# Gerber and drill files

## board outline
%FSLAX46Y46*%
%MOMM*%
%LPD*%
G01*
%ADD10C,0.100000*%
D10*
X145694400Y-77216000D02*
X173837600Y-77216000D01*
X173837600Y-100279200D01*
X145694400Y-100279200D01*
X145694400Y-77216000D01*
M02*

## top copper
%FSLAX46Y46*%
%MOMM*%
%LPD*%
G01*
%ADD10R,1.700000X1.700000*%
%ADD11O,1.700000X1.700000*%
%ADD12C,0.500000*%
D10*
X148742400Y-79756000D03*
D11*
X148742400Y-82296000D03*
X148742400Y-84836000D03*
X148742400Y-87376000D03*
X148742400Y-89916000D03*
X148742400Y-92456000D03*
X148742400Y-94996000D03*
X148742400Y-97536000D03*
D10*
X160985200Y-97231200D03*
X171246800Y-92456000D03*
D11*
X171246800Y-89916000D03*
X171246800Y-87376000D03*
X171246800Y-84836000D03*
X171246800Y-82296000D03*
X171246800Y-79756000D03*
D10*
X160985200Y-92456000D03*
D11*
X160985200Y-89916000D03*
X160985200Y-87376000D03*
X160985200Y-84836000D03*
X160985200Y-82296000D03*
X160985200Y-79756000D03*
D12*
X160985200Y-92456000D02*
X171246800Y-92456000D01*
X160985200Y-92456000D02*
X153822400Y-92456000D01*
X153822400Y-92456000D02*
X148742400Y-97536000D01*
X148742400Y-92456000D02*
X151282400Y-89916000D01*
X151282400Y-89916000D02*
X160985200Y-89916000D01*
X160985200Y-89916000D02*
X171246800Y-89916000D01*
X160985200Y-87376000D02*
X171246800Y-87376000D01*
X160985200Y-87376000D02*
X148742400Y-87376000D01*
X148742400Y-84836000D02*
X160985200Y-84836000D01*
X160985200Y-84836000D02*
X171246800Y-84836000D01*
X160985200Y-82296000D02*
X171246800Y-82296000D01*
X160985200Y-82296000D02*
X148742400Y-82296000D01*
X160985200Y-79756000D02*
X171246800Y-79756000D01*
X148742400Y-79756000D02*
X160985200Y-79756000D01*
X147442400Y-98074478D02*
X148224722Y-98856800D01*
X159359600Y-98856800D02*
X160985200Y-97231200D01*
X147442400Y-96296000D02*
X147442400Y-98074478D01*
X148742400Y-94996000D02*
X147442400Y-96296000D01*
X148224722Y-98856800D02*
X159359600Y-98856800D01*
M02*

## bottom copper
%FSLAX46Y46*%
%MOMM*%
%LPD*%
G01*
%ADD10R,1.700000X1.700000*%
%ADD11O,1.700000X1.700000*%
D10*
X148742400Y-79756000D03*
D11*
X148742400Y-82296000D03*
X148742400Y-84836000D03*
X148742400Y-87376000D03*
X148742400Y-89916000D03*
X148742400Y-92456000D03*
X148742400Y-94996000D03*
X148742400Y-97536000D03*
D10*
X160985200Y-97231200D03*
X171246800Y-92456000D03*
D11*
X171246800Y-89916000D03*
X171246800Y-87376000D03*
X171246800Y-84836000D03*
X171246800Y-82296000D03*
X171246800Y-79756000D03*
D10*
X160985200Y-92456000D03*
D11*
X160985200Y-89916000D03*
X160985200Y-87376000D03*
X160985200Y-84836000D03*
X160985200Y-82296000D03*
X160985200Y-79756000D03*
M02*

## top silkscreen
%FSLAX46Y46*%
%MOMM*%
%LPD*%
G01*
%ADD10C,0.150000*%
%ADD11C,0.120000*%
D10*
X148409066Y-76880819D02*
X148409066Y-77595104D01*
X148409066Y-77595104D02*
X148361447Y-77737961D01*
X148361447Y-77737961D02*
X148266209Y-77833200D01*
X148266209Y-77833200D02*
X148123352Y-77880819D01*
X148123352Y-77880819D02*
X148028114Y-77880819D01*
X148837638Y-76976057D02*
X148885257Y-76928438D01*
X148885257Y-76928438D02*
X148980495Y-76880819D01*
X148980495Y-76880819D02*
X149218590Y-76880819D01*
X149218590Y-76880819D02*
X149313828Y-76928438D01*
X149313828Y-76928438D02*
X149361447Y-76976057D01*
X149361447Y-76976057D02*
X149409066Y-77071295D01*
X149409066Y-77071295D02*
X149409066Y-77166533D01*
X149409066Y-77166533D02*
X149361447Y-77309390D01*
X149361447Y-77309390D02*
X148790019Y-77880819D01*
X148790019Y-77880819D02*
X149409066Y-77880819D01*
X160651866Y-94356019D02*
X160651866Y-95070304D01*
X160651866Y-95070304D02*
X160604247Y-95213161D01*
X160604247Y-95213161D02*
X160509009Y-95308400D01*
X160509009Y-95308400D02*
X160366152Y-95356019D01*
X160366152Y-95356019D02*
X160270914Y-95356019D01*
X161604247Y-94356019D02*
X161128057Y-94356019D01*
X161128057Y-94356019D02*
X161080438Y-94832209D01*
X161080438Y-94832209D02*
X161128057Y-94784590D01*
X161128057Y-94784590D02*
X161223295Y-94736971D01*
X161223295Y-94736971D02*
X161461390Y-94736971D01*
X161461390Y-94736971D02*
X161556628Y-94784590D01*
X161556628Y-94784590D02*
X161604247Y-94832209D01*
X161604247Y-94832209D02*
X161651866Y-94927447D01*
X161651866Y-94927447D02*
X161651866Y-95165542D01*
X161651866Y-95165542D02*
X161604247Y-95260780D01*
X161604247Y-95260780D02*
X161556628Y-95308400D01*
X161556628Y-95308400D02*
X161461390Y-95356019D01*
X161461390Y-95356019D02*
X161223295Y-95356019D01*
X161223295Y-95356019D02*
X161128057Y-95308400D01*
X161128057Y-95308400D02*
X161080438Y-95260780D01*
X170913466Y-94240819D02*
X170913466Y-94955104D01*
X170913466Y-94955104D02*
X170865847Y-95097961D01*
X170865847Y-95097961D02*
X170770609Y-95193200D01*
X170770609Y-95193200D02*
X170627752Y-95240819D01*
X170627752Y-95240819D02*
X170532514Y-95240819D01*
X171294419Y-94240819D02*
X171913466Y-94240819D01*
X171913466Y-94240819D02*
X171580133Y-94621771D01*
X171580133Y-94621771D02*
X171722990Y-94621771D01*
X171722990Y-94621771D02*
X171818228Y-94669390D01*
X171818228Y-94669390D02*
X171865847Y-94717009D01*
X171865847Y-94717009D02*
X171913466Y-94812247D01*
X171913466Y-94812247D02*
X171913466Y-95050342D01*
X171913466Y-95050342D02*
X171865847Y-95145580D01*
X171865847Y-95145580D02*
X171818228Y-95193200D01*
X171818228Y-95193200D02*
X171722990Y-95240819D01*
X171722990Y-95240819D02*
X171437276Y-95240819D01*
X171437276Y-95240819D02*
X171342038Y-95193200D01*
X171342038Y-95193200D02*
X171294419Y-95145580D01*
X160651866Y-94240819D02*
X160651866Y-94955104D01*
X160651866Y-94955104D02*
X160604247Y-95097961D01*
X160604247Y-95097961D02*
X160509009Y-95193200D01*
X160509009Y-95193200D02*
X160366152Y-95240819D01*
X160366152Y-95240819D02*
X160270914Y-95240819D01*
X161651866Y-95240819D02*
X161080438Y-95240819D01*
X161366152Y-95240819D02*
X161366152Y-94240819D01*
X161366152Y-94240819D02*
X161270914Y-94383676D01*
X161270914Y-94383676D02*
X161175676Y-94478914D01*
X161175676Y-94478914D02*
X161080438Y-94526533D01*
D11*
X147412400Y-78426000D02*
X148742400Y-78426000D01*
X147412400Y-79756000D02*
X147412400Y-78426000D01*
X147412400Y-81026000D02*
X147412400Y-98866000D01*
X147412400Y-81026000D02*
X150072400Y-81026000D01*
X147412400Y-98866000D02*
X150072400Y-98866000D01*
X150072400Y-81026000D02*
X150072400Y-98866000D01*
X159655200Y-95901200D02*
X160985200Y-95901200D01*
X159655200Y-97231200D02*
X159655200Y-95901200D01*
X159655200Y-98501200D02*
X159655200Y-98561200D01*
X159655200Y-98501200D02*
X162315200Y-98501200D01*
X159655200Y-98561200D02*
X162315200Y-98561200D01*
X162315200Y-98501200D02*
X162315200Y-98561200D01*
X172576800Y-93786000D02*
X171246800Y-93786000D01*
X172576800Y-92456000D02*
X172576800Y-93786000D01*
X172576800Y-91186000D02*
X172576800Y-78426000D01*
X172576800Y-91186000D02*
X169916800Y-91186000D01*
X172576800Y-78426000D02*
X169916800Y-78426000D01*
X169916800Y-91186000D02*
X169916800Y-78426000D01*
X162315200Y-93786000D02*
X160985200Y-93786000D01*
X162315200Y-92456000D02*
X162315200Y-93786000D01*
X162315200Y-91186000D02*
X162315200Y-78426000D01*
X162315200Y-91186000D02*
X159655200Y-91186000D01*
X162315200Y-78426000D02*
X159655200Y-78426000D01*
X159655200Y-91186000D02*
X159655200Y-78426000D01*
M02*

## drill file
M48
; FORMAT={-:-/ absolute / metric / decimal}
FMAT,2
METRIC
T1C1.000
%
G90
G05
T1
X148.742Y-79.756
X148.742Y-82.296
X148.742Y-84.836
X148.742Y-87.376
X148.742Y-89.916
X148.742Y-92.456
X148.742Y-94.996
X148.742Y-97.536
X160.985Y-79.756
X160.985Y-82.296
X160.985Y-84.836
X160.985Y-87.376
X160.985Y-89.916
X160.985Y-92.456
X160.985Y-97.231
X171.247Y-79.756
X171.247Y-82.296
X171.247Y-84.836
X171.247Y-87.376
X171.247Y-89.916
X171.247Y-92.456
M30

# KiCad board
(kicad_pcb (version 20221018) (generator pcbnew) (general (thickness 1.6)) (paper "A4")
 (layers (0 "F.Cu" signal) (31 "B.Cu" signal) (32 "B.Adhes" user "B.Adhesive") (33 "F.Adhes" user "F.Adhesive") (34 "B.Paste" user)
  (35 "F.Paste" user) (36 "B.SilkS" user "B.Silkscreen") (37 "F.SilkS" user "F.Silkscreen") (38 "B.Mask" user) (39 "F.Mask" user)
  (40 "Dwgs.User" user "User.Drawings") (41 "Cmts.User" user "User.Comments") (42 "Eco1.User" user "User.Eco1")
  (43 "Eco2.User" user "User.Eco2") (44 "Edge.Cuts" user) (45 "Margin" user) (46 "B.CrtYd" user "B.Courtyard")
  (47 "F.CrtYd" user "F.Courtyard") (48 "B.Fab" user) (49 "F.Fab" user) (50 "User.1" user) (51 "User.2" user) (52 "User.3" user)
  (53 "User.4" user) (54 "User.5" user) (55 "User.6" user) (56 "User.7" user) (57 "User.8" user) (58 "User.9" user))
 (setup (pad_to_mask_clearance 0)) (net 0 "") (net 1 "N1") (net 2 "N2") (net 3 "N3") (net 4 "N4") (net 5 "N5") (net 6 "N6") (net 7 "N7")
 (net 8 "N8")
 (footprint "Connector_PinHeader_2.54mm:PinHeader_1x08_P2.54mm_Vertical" (layer "F.Cu") (at 148.7424 79.756)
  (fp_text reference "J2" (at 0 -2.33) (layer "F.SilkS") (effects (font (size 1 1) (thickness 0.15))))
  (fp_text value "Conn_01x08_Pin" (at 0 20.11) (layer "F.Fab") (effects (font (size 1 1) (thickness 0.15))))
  (fp_line (start -1.33 -1.33) (end 0 -1.33) (stroke (width 0.12) (type solid)) (layer "F.SilkS"))
  (fp_line (start -1.33 0) (end -1.33 -1.33) (stroke (width 0.12) (type solid)) (layer "F.SilkS"))
  (fp_line (start -1.33 1.27) (end -1.33 19.11) (stroke (width 0.12) (type solid)) (layer "F.SilkS"))
  (fp_line (start -1.33 1.27) (end 1.33 1.27) (stroke (width 0.12) (type solid)) (layer "F.SilkS"))
  (fp_line (start -1.33 19.11) (end 1.33 19.11) (stroke (width 0.12) (type solid)) (layer "F.SilkS"))
  (fp_line (start 1.33 1.27) (end 1.33 19.11) (stroke (width 0.12) (type solid)) (layer "F.SilkS"))
  (pad "1" thru_hole rect (at 0 0) (size 1.7 1.7) (drill 1) (layers "*.Cu" "*.Mask") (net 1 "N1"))
  (pad "2" thru_hole oval (at 0 2.54) (size 1.7 1.7) (drill 1) (layers "*.Cu" "*.Mask") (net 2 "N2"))
  (pad "3" thru_hole oval (at 0 5.08) (size 1.7 1.7) (drill 1) (layers "*.Cu" "*.Mask") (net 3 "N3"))
  (pad "4" thru_hole oval (at 0 7.62) (size 1.7 1.7) (drill 1) (layers "*.Cu" "*.Mask") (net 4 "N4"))
  (pad "5" thru_hole oval (at 0 10.16) (size 1.7 1.7) (drill 1) (layers "*.Cu" "*.Mask") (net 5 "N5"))
  (pad "6" thru_hole oval (at 0 12.7) (size 1.7 1.7) (drill 1) (layers "*.Cu" "*.Mask") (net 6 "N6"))
  (pad "7" thru_hole oval (at 0 15.24) (size 1.7 1.7) (drill 1) (layers "*.Cu" "*.Mask") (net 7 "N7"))
  (pad "8" thru_hole oval (at 0 17.78) (size 1.7 1.7) (drill 1) (layers "*.Cu" "*.Mask") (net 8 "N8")))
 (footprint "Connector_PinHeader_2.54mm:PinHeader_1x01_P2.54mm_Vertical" (layer "F.Cu") (at 160.9852 97.2312)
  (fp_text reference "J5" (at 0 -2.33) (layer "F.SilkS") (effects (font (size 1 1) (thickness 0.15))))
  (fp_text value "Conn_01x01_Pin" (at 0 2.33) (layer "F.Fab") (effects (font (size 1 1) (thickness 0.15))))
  (fp_line (start -1.33 -1.33) (end 0 -1.33) (stroke (width 0.12) (type solid)) (layer "F.SilkS"))
  (fp_line (start -1.33 0) (end -1.33 -1.33) (stroke (width 0.12) (type solid)) (layer "F.SilkS"))
  (fp_line (start -1.33 1.27) (end -1.33 1.33) (stroke (width 0.12) (type solid)) (layer "F.SilkS"))
  (fp_line (start -1.33 1.27) (end 1.33 1.27) (stroke (width 0.12) (type solid)) (layer "F.SilkS"))
  (fp_line (start -1.33 1.33) (end 1.33 1.33) (stroke (width 0.12) (type solid)) (layer "F.SilkS"))
  (fp_line (start 1.33 1.27) (end 1.33 1.33) (stroke (width 0.12) (type solid)) (layer "F.SilkS"))
  (pad "1" thru_hole rect (at 0 0) (size 1.7 1.7) (drill 1) (layers "*.Cu" "*.Mask") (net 7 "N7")))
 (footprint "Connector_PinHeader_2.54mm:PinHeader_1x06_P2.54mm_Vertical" (layer "F.Cu") (at 171.2468 92.456 180)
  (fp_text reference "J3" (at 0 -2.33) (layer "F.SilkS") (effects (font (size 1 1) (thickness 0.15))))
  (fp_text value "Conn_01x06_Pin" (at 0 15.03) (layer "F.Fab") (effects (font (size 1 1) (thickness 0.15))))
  (fp_line (start -1.33 -1.33) (end 0 -1.33) (stroke (width 0.12) (type solid)) (layer "F.SilkS"))
  (fp_line (start -1.33 0) (end -1.33 -1.33) (stroke (width 0.12) (type solid)) (layer "F.SilkS"))
  (fp_line (start -1.33 1.27) (end -1.33 14.03) (stroke (width 0.12) (type solid)) (layer "F.SilkS"))
  (fp_line (start -1.33 1.27) (end 1.33 1.27) (stroke (width 0.12) (type solid)) (layer "F.SilkS"))
  (fp_line (start -1.33 14.03) (end 1.33 14.03) (stroke (width 0.12) (type solid)) (layer "F.SilkS"))
  (fp_line (start 1.33 1.27) (end 1.33 14.03) (stroke (width 0.12) (type solid)) (layer "F.SilkS"))
  (pad "1" thru_hole rect (at 0 0 180) (size 1.7 1.7) (drill 1) (layers "*.Cu" "*.Mask") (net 8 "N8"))
  (pad "2" thru_hole oval (at 0 2.54 180) (size 1.7 1.7) (drill 1) (layers "*.Cu" "*.Mask") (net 6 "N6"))
  (pad "3" thru_hole oval (at 0 5.08 180) (size 1.7 1.7) (drill 1) (layers "*.Cu" "*.Mask") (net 4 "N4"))
  (pad "4" thru_hole oval (at 0 7.62 180) (size 1.7 1.7) (drill 1) (layers "*.Cu" "*.Mask") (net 3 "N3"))
  (pad "5" thru_hole oval (at 0 10.16 180) (size 1.7 1.7) (drill 1) (layers "*.Cu" "*.Mask") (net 2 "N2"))
  (pad "6" thru_hole oval (at 0 12.7 180) (size 1.7 1.7) (drill 1) (layers "*.Cu" "*.Mask") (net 1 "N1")))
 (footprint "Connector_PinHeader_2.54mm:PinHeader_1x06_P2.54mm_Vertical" (layer "F.Cu") (at 160.9852 92.456 180)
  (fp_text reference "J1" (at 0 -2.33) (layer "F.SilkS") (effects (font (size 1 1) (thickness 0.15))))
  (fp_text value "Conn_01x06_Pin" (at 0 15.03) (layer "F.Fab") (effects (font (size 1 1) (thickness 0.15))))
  (fp_line (start -1.33 -1.33) (end 0 -1.33) (stroke (width 0.12) (type solid)) (layer "F.SilkS"))
  (fp_line (start -1.33 0) (end -1.33 -1.33) (stroke (width 0.12) (type solid)) (layer "F.SilkS"))
  (fp_line (start -1.33 1.27) (end -1.33 14.03) (stroke (width 0.12) (type solid)) (layer "F.SilkS"))
  (fp_line (start -1.33 1.27) (end 1.33 1.27) (stroke (width 0.12) (type solid)) (layer "F.SilkS"))
  (fp_line (start -1.33 14.03) (end 1.33 14.03) (stroke (width 0.12) (type solid)) (layer "F.SilkS"))
  (fp_line (start 1.33 1.27) (end 1.33 14.03) (stroke (width 0.12) (type solid)) (layer "F.SilkS"))
  (pad "1" thru_hole rect (at 0 0 180) (size 1.7 1.7) (drill 1) (layers "*.Cu" "*.Mask") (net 8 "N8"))
  (pad "2" thru_hole oval (at 0 2.54 180) (size 1.7 1.7) (drill 1) (layers "*.Cu" "*.Mask") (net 6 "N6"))
  (pad "3" thru_hole oval (at 0 5.08 180) (size 1.7 1.7) (drill 1) (layers "*.Cu" "*.Mask") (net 4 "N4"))
  (pad "4" thru_hole oval (at 0 7.62 180) (size 1.7 1.7) (drill 1) (layers "*.Cu" "*.Mask") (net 3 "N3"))
  (pad "5" thru_hole oval (at 0 10.16 180) (size 1.7 1.7) (drill 1) (layers "*.Cu" "*.Mask") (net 2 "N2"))
  (pad "6" thru_hole oval (at 0 12.7 180) (size 1.7 1.7) (drill 1) (layers "*.Cu" "*.Mask") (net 1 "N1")))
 (gr_rect (start 145.6944 77.216) (end 173.8376 100.2792) (stroke (width 0.1) (type default)) (fill none) (layer "Edge.Cuts"))
 (segment (start 160.9852 92.456) (end 171.2468 92.456) (width 0.5) (layer "F.Cu") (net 8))
 (segment (start 160.9852 92.456) (end 153.8224 92.456) (width 0.5) (layer "F.Cu") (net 8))
 (segment (start 153.8224 92.456) (end 148.7424 97.536) (width 0.5) (layer "F.Cu") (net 8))
 (segment (start 148.7424 92.456) (end 151.2824 89.916) (width 0.5) (layer "F.Cu") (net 6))
 (segment (start 151.2824 89.916) (end 160.9852 89.916) (width 0.5) (layer "F.Cu") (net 6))
 (segment (start 160.9852 89.916) (end 171.2468 89.916) (width 0.5) (layer "F.Cu") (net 6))
 (segment (start 160.9852 87.376) (end 171.2468 87.376) (width 0.5) (layer "F.Cu") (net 4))
 (segment (start 160.9852 87.376) (end 148.7424 87.376) (width 0.5) (layer "F.Cu") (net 4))
 (segment (start 148.7424 84.836) (end 160.9852 84.836) (width 0.5) (layer "F.Cu") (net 3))
 (segment (start 160.9852 84.836) (end 171.2468 84.836) (width 0.5) (layer "F.Cu") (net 3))
 (segment (start 160.9852 82.296) (end 171.2468 82.296) (width 0.5) (layer "F.Cu") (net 2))
 (segment (start 160.9852 82.296) (end 148.7424 82.296) (width 0.5) (layer "F.Cu") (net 2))
 (segment (start 160.9852 79.756) (end 171.2468 79.756) (width 0.5) (layer "F.Cu") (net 1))
 (segment (start 148.7424 79.756) (end 160.9852 79.756) (width 0.5) (layer "F.Cu") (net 1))
 (segment (start 147.4424 98.074478) (end 148.224722 98.8568) (width 0.5) (layer "F.Cu") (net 7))
 (segment (start 159.3596 98.8568) (end 160.9852 97.2312) (width 0.5) (layer "F.Cu") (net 7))
 (segment (start 147.4424 96.296) (end 147.4424 98.074478) (width 0.5) (layer "F.Cu") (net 7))
 (segment (start 148.7424 94.996) (end 147.4424 96.296) (width 0.5) (layer "F.Cu") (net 7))
 (segment (start 148.224722 98.8568) (end 159.3596 98.8568) (width 0.5) (layer "F.Cu") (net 7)))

